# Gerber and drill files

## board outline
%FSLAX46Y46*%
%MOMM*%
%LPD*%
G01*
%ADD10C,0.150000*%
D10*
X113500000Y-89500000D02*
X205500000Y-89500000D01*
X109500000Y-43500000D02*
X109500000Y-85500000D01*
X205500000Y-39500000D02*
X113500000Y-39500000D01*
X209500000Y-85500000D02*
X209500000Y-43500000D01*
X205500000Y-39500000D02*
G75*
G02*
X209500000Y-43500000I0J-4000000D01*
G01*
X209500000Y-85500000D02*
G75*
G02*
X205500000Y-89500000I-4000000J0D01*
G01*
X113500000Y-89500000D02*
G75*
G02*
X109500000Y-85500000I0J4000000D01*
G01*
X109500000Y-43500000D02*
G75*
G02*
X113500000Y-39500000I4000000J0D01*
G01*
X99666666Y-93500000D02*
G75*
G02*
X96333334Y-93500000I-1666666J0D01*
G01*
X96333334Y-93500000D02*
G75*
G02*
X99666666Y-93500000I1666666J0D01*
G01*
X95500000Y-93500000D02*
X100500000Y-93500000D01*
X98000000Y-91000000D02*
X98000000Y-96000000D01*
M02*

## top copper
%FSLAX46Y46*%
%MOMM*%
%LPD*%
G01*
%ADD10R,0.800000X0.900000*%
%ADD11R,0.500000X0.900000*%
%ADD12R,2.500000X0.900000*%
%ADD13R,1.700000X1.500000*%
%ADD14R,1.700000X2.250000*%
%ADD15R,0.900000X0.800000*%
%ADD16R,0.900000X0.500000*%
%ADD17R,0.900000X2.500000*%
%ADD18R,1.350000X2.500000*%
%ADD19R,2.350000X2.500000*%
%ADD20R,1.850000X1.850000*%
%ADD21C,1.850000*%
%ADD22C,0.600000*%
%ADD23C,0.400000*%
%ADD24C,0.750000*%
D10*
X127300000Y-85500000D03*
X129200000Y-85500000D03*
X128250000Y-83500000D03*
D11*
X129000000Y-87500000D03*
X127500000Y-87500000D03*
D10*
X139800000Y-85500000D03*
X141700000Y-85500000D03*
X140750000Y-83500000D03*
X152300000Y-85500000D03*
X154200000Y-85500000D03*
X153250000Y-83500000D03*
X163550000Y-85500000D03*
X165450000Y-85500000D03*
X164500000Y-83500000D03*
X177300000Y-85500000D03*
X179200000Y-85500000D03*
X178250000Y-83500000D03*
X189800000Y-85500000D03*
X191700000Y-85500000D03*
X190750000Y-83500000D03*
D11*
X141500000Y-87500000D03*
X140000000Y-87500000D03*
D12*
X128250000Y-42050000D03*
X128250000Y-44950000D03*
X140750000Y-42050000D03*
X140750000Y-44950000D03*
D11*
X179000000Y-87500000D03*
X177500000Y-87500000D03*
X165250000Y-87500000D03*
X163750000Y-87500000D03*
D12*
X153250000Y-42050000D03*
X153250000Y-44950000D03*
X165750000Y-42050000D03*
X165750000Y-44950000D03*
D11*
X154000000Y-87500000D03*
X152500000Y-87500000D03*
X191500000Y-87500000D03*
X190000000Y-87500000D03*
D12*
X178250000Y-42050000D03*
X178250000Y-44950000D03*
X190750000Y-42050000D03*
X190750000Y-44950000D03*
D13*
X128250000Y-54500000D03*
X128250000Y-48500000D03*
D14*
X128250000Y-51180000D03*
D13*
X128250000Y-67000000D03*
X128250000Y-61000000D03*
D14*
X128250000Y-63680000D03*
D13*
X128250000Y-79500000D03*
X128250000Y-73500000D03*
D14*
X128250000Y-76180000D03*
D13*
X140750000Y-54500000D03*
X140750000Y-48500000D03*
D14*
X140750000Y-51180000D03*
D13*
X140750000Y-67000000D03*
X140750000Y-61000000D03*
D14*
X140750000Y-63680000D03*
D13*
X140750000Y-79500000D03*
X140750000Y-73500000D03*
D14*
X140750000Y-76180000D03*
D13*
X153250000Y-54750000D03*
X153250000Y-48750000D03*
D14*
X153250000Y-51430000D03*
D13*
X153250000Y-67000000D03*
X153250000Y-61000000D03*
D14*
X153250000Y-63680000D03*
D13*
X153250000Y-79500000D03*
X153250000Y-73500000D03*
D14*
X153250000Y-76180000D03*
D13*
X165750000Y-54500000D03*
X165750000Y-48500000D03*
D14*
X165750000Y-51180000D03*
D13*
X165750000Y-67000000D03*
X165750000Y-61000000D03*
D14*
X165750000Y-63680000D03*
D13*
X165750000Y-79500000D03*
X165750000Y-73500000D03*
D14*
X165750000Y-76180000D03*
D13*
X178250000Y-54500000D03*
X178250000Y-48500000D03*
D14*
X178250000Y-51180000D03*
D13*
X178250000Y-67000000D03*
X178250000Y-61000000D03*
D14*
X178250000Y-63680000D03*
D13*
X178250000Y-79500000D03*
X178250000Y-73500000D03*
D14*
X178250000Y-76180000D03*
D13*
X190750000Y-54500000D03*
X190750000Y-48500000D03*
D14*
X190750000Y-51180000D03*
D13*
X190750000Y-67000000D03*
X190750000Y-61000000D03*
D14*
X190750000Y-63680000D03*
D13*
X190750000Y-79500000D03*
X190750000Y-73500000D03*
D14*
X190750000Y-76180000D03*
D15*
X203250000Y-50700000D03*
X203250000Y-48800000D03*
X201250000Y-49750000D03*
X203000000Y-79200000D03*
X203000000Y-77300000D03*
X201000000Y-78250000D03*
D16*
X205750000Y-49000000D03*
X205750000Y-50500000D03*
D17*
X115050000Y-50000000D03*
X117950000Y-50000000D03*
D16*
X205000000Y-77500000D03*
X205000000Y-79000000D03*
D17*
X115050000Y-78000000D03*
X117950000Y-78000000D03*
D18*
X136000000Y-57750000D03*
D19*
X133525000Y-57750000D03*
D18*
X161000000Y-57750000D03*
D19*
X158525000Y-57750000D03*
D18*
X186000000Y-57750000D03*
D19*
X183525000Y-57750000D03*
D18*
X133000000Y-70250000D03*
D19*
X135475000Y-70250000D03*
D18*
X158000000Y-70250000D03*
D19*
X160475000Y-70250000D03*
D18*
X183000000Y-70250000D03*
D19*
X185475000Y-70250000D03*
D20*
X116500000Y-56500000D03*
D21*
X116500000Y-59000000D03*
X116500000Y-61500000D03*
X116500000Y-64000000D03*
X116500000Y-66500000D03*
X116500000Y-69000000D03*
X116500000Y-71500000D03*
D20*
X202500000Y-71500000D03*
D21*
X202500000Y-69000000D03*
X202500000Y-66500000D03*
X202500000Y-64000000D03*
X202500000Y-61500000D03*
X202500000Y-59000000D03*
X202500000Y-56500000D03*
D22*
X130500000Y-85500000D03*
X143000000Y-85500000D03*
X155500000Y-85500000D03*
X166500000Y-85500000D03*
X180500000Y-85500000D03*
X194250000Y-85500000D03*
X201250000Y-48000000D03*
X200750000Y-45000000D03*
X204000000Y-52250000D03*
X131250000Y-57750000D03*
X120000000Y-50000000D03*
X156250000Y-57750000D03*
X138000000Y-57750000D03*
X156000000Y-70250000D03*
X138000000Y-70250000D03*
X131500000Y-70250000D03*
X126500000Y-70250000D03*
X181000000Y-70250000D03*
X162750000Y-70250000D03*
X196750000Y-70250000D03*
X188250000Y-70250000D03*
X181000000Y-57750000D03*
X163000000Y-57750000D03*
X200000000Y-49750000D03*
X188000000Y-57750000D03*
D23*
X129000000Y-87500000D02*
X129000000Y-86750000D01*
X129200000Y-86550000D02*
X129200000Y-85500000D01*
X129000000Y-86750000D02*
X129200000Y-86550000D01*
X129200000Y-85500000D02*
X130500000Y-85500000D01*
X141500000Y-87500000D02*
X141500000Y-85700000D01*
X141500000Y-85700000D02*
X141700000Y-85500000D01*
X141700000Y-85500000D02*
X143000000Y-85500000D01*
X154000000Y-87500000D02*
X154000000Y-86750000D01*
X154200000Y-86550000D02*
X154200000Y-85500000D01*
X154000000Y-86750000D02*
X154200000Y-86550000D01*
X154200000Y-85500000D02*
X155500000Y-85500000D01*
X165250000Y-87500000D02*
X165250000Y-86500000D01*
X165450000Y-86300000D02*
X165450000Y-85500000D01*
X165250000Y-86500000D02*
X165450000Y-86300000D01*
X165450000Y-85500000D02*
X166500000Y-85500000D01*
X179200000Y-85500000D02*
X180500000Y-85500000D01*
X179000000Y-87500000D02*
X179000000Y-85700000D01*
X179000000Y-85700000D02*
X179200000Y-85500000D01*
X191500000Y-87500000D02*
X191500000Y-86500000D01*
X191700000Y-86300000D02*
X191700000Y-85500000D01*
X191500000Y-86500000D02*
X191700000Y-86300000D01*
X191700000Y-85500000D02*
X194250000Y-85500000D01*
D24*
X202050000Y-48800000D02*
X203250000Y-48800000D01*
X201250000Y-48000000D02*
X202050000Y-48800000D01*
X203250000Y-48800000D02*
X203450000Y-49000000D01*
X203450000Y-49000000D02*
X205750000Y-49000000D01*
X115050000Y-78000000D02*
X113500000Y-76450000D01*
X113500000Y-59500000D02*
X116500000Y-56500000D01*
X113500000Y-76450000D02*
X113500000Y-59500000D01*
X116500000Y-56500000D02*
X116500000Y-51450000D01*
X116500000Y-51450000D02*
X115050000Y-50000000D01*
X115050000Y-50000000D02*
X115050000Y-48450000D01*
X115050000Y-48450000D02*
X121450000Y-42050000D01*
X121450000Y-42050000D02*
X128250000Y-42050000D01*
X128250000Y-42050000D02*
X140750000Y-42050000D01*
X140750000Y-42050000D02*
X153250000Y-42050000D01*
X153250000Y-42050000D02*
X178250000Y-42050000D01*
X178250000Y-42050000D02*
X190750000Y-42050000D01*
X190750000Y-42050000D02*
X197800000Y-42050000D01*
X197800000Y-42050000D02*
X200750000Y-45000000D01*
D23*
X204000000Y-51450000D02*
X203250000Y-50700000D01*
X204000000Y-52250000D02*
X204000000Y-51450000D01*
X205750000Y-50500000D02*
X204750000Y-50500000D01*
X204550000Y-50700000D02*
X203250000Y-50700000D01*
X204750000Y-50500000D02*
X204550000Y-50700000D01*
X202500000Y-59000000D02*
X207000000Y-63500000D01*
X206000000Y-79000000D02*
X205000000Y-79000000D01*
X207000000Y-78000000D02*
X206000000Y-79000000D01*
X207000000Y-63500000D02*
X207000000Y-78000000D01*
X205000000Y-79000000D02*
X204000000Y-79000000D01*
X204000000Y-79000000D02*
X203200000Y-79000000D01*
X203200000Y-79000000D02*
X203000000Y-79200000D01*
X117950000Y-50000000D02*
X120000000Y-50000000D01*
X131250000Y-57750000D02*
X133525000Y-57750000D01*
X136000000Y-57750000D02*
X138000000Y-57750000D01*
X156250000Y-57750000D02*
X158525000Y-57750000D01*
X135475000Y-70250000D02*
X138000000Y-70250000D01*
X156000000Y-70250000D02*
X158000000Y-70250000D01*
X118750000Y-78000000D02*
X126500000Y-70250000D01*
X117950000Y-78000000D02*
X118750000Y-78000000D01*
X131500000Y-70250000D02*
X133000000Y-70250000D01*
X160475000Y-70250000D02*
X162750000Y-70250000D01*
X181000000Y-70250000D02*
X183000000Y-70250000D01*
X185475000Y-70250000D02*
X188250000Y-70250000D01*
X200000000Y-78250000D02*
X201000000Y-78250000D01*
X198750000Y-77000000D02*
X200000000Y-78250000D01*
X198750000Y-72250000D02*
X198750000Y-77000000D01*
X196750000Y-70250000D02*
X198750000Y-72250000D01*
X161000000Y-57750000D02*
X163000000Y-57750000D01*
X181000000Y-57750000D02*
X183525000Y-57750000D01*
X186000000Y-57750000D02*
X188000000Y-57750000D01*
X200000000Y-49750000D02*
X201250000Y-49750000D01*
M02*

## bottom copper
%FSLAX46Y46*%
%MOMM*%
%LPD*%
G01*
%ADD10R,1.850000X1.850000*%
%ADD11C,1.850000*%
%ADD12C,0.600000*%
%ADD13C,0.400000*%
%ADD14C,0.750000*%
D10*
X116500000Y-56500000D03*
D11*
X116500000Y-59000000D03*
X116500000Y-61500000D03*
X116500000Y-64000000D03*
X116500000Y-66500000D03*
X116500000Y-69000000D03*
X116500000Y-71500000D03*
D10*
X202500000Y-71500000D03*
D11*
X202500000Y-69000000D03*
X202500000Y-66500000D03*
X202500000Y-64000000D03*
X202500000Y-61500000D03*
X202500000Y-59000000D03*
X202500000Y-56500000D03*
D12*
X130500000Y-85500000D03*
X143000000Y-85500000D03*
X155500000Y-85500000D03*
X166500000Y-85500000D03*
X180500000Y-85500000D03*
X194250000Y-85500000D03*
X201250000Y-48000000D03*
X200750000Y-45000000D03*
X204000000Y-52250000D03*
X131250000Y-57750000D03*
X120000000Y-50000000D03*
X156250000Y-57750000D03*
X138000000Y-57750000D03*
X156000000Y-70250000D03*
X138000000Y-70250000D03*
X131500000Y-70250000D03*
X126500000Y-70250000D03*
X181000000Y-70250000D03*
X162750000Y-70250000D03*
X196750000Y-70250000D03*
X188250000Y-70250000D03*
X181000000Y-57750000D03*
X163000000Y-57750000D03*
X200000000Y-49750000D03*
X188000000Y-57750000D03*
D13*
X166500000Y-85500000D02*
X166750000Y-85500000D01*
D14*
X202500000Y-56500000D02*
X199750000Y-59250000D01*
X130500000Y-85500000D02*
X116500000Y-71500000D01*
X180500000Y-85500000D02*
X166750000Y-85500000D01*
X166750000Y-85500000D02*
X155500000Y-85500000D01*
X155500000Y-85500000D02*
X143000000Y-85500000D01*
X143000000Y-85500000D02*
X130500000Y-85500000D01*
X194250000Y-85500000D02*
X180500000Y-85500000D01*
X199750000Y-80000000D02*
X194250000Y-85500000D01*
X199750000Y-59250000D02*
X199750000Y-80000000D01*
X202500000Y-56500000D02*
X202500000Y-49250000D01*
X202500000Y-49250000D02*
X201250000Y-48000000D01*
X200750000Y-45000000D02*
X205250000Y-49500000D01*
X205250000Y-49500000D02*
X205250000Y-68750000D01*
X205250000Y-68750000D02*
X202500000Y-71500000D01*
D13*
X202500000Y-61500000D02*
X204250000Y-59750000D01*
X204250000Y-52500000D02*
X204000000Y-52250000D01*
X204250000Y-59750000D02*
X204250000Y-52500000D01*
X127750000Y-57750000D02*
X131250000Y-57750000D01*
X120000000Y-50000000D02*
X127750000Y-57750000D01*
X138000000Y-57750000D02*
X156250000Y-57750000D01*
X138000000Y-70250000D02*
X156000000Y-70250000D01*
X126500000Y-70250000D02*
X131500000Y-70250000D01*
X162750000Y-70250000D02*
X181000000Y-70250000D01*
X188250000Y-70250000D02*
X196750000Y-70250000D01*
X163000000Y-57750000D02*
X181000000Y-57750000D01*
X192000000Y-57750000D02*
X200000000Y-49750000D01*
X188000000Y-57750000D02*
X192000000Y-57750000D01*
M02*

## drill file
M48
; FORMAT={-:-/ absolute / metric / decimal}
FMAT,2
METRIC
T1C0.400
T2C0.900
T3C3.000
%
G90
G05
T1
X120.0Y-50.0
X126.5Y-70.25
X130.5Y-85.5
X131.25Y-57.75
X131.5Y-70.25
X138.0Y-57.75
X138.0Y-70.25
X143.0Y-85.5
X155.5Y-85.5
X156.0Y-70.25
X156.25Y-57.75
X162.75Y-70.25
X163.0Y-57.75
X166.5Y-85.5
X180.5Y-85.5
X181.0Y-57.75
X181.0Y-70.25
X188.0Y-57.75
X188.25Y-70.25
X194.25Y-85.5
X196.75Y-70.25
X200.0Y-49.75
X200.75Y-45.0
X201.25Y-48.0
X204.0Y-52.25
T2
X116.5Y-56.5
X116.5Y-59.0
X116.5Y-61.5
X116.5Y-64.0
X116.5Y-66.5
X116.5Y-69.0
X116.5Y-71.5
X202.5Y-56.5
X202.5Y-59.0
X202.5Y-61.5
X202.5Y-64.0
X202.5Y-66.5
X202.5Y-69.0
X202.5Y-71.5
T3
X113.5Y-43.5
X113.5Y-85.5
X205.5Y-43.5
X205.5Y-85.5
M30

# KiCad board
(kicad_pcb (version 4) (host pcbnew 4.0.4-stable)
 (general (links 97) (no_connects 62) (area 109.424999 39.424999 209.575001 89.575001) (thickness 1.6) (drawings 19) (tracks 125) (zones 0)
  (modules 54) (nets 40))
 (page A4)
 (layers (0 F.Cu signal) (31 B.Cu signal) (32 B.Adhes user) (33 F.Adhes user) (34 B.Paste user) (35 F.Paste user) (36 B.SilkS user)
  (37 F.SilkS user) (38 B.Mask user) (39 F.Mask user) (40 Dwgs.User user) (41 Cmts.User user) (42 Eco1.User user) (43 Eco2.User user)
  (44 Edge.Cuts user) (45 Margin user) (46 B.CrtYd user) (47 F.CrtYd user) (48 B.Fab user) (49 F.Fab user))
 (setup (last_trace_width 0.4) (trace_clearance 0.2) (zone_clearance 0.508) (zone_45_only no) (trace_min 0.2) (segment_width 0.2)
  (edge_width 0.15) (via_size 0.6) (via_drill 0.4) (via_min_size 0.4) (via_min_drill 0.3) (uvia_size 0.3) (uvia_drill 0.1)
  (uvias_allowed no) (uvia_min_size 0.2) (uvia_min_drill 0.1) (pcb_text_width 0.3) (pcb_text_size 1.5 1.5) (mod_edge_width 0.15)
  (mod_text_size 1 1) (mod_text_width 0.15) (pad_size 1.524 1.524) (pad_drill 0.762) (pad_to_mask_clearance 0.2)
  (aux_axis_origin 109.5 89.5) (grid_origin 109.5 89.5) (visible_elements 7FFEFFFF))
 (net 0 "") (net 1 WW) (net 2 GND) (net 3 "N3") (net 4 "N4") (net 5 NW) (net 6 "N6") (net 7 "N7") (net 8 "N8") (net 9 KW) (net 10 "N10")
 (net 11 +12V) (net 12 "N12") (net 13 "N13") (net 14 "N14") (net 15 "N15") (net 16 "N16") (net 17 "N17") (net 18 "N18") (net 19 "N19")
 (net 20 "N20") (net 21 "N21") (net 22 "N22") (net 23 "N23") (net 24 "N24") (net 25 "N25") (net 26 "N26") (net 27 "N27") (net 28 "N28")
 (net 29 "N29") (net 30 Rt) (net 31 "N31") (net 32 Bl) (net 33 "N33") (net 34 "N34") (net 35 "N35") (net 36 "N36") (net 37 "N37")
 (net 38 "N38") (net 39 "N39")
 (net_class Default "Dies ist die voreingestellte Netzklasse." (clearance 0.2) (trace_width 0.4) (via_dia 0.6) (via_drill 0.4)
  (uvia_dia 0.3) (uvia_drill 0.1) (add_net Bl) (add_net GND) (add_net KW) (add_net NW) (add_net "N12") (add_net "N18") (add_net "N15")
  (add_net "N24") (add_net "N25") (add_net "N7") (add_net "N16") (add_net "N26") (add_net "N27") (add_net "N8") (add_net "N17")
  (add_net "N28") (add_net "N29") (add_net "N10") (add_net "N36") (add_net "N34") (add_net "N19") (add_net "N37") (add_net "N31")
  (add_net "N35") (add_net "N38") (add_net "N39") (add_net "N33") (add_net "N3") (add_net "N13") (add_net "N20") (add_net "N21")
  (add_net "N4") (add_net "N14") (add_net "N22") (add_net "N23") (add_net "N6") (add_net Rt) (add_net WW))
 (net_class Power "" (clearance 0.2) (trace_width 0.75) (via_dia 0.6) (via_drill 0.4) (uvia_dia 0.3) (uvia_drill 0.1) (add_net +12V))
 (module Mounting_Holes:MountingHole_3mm (layer F.Cu) (at 205.5 85.5)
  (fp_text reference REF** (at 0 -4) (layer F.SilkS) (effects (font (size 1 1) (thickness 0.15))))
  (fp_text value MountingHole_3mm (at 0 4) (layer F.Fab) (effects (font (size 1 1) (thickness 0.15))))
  (pad 1 np_thru_hole circle (at 0 0) (size 3 3) (drill 3) (layers *.Cu *.Mask)))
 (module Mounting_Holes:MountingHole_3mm (layer F.Cu) (at 205.5 43.5)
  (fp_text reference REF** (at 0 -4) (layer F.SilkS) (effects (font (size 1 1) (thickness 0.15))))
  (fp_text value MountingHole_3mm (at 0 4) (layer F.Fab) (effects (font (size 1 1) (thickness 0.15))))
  (pad 1 np_thru_hole circle (at 0 0) (size 3 3) (drill 3) (layers *.Cu *.Mask)))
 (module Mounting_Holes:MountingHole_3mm (layer F.Cu) (at 113.5 85.5)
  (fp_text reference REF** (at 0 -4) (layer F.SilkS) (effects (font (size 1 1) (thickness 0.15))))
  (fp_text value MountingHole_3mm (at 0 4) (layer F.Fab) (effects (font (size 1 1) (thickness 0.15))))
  (pad 1 np_thru_hole circle (at 0 0) (size 3 3) (drill 3) (layers *.Cu *.Mask)))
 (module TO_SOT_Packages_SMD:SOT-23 (layer F.Cu) (at 128.25 84.5 90)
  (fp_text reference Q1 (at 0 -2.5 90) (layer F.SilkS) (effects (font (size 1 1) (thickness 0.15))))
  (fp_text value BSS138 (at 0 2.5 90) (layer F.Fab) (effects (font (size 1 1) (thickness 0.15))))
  (pad 1 smd rect (at -1 -0.95 90) (size 0.9 0.8) (layers F.Cu F.Paste F.Mask) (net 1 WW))
  (pad 2 smd rect (at -1 0.95 90) (size 0.9 0.8) (layers F.Cu F.Paste F.Mask) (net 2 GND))
  (pad 3 smd rect (at 1 0 90) (size 0.9 0.8) (layers F.Cu F.Paste F.Mask) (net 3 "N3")))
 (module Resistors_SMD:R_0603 (layer F.Cu) (at 128.25 87.5 180)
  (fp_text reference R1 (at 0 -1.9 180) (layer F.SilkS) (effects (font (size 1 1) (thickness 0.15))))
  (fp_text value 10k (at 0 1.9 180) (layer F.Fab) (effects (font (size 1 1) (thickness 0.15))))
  (pad 1 smd rect (at -0.75 0 180) (size 0.5 0.9) (layers F.Cu F.Paste F.Mask) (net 2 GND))
  (pad 2 smd rect (at 0.75 0 180) (size 0.5 0.9) (layers F.Cu F.Paste F.Mask) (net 1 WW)))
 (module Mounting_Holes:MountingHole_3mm (layer F.Cu) (at 113.5 43.5)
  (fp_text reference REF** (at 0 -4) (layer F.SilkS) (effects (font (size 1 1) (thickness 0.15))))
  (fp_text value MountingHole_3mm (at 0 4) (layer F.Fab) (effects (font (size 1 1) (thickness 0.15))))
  (pad 1 np_thru_hole circle (at 0 0) (size 3 3) (drill 3) (layers *.Cu *.Mask)))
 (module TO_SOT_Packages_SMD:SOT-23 (layer F.Cu) (at 140.75 84.5 90)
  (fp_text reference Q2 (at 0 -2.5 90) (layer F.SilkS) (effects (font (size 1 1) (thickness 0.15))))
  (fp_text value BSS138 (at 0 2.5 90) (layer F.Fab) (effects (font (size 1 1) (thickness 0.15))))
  (pad 1 smd rect (at -1 -0.95 90) (size 0.9 0.8) (layers F.Cu F.Paste F.Mask) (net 1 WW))
  (pad 2 smd rect (at -1 0.95 90) (size 0.9 0.8) (layers F.Cu F.Paste F.Mask) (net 2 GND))
  (pad 3 smd rect (at 1 0 90) (size 0.9 0.8) (layers F.Cu F.Paste F.Mask) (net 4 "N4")))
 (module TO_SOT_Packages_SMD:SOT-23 (layer F.Cu) (at 153.25 84.5 90)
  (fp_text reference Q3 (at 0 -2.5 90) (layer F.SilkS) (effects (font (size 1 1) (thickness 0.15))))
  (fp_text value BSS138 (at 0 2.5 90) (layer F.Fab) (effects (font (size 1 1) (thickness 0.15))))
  (pad 1 smd rect (at -1 -0.95 90) (size 0.9 0.8) (layers F.Cu F.Paste F.Mask) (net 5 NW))
  (pad 2 smd rect (at -1 0.95 90) (size 0.9 0.8) (layers F.Cu F.Paste F.Mask) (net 2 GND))
  (pad 3 smd rect (at 1 0 90) (size 0.9 0.8) (layers F.Cu F.Paste F.Mask) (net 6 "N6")))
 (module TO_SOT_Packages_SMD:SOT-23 (layer F.Cu) (at 164.5 84.5 90)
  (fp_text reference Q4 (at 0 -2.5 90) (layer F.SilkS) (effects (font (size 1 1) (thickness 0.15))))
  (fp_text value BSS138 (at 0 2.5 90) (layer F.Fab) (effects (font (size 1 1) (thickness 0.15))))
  (pad 1 smd rect (at -1 -0.95 90) (size 0.9 0.8) (layers F.Cu F.Paste F.Mask) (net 5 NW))
  (pad 2 smd rect (at -1 0.95 90) (size 0.9 0.8) (layers F.Cu F.Paste F.Mask) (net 2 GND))
  (pad 3 smd rect (at 1 0 90) (size 0.9 0.8) (layers F.Cu F.Paste F.Mask) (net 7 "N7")))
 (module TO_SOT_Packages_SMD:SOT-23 (layer F.Cu) (at 178.25 84.5 90)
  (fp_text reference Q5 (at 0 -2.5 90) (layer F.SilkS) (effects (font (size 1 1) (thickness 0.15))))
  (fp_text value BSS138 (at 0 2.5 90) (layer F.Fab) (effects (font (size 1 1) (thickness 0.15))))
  (pad 1 smd rect (at -1 -0.95 90) (size 0.9 0.8) (layers F.Cu F.Paste F.Mask) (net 5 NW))
  (pad 2 smd rect (at -1 0.95 90) (size 0.9 0.8) (layers F.Cu F.Paste F.Mask) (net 2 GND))
  (pad 3 smd rect (at 1 0 90) (size 0.9 0.8) (layers F.Cu F.Paste F.Mask) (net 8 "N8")))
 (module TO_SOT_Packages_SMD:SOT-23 (layer F.Cu) (at 190.75 84.5 90)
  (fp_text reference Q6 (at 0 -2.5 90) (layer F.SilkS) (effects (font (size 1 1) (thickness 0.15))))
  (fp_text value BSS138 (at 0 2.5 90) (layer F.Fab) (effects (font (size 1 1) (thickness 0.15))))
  (pad 1 smd rect (at -1 -0.95 90) (size 0.9 0.8) (layers F.Cu F.Paste F.Mask) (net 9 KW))
  (pad 2 smd rect (at -1 0.95 90) (size 0.9 0.8) (layers F.Cu F.Paste F.Mask) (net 2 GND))
  (pad 3 smd rect (at 1 0 90) (size 0.9 0.8) (layers F.Cu F.Paste F.Mask) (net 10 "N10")))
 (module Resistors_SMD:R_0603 (layer F.Cu) (at 140.75 87.5 180)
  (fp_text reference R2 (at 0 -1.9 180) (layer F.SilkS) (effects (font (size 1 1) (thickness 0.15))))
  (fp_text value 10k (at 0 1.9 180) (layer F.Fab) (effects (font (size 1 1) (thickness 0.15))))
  (pad 1 smd rect (at -0.75 0 180) (size 0.5 0.9) (layers F.Cu F.Paste F.Mask) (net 2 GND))
  (pad 2 smd rect (at 0.75 0 180) (size 0.5 0.9) (layers F.Cu F.Paste F.Mask) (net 1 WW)))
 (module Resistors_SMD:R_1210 (layer F.Cu) (at 128.25 43.5 270)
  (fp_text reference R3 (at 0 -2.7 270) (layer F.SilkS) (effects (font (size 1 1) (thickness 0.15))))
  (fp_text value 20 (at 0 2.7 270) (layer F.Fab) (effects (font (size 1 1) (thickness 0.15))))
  (pad 1 smd rect (at -1.45 0 270) (size 0.9 2.5) (layers F.Cu F.Paste F.Mask) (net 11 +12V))
  (pad 2 smd rect (at 1.45 0 270) (size 0.9 2.5) (layers F.Cu F.Paste F.Mask) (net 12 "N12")))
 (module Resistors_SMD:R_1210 (layer F.Cu) (at 140.75 43.5 270)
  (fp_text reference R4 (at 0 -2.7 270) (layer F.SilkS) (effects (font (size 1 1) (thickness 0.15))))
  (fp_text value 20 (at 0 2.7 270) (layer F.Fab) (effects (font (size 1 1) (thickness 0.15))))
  (pad 1 smd rect (at -1.45 0 270) (size 0.9 2.5) (layers F.Cu F.Paste F.Mask) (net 11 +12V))
  (pad 2 smd rect (at 1.45 0 270) (size 0.9 2.5) (layers F.Cu F.Paste F.Mask) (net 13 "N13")))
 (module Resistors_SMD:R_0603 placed (layer F.Cu) (at 178.25 87.5 180)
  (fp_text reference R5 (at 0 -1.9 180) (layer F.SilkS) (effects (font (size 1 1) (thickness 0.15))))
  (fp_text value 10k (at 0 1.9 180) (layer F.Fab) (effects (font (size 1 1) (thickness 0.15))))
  (pad 1 smd rect (at -0.75 0 180) (size 0.5 0.9) (layers F.Cu F.Paste F.Mask) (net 2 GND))
  (pad 2 smd rect (at 0.75 0 180) (size 0.5 0.9) (layers F.Cu F.Paste F.Mask) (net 5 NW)))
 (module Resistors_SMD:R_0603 (layer F.Cu) (at 164.5 87.5 180)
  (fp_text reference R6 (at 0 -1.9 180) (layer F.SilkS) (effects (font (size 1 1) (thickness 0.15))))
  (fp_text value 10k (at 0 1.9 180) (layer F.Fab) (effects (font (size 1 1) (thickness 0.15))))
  (pad 1 smd rect (at -0.75 0 180) (size 0.5 0.9) (layers F.Cu F.Paste F.Mask) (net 2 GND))
  (pad 2 smd rect (at 0.75 0 180) (size 0.5 0.9) (layers F.Cu F.Paste F.Mask) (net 5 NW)))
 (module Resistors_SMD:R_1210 (layer F.Cu) (at 153.25 43.5 270)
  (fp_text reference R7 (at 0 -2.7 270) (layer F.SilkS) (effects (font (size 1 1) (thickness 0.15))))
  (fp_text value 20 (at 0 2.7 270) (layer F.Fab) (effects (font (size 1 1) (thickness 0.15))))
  (pad 1 smd rect (at -1.45 0 270) (size 0.9 2.5) (layers F.Cu F.Paste F.Mask) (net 11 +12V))
  (pad 2 smd rect (at 1.45 0 270) (size 0.9 2.5) (layers F.Cu F.Paste F.Mask) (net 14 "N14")))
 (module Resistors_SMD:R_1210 (layer F.Cu) (at 165.75 43.5 270)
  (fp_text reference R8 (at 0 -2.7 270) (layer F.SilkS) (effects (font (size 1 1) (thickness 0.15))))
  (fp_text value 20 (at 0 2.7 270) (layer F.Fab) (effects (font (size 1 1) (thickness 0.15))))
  (pad 1 smd rect (at -1.45 0 270) (size 0.9 2.5) (layers F.Cu F.Paste F.Mask) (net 11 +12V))
  (pad 2 smd rect (at 1.45 0 270) (size 0.9 2.5) (layers F.Cu F.Paste F.Mask) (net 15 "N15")))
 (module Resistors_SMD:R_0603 (layer F.Cu) (at 153.25 87.5 180)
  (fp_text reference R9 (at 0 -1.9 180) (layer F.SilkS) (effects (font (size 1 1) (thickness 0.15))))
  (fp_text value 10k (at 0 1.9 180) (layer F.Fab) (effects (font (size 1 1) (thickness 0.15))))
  (pad 1 smd rect (at -0.75 0 180) (size 0.5 0.9) (layers F.Cu F.Paste F.Mask) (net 2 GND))
  (pad 2 smd rect (at 0.75 0 180) (size 0.5 0.9) (layers F.Cu F.Paste F.Mask) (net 5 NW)))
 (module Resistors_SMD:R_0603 (layer F.Cu) (at 190.75 87.5 180)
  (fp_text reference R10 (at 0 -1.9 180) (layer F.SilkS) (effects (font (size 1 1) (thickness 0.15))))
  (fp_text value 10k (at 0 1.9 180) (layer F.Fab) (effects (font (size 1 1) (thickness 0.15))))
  (pad 1 smd rect (at -0.75 0 180) (size 0.5 0.9) (layers F.Cu F.Paste F.Mask) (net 2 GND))
  (pad 2 smd rect (at 0.75 0 180) (size 0.5 0.9) (layers F.Cu F.Paste F.Mask) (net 9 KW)))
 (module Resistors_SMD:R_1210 (layer F.Cu) (at 178.25 43.5 270)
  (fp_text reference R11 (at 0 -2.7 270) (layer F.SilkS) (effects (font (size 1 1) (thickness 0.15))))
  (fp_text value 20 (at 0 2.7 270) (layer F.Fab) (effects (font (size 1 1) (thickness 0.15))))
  (pad 1 smd rect (at -1.45 0 270) (size 0.9 2.5) (layers F.Cu F.Paste F.Mask) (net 11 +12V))
  (pad 2 smd rect (at 1.45 0 270) (size 0.9 2.5) (layers F.Cu F.Paste F.Mask) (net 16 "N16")))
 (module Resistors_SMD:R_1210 (layer F.Cu) (at 190.75 43.5 270)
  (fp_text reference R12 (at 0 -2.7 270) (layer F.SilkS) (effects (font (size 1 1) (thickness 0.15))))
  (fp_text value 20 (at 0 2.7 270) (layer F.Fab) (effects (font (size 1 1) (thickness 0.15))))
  (pad 1 smd rect (at -1.45 0 270) (size 0.9 2.5) (layers F.Cu F.Paste F.Mask) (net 11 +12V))
  (pad 2 smd rect (at 1.45 0 270) (size 0.9 2.5) (layers F.Cu F.Paste F.Mask) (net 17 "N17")))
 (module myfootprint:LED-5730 (layer F.Cu) (at 128.25 51.5 90)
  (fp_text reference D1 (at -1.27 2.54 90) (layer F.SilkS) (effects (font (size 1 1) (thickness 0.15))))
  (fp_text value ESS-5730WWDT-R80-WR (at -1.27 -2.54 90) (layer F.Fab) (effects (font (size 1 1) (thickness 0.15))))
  (pad 2 smd rect (at -3 0 90) (size 1.5 1.7) (layers F.Cu F.Paste F.Mask) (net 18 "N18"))
  (pad 1 smd rect (at 3 0 90) (size 1.5 1.7) (layers F.Cu F.Paste F.Mask) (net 12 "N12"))
  (pad 1 smd rect (at 0.32 0 90) (size 2.25 1.7) (layers F.Cu F.Paste F.Mask) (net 12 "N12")))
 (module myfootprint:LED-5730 (layer F.Cu) (at 128.25 64 90)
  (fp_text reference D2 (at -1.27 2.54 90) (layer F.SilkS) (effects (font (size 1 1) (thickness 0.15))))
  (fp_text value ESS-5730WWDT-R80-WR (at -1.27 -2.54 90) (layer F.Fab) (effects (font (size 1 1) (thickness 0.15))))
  (pad 2 smd rect (at -3 0 90) (size 1.5 1.7) (layers F.Cu F.Paste F.Mask) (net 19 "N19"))
  (pad 1 smd rect (at 3 0 90) (size 1.5 1.7) (layers F.Cu F.Paste F.Mask) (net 18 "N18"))
  (pad 1 smd rect (at 0.32 0 90) (size 2.25 1.7) (layers F.Cu F.Paste F.Mask) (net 18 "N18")))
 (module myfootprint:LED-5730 (layer F.Cu) (at 128.25 76.5 90)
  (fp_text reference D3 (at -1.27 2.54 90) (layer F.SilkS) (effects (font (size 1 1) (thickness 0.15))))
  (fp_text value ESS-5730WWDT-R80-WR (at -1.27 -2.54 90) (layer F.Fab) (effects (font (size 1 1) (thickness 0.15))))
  (pad 2 smd rect (at -3 0 90) (size 1.5 1.7) (layers F.Cu F.Paste F.Mask) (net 3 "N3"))
  (pad 1 smd rect (at 3 0 90) (size 1.5 1.7) (layers F.Cu F.Paste F.Mask) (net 19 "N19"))
  (pad 1 smd rect (at 0.32 0 90) (size 2.25 1.7) (layers F.Cu F.Paste F.Mask) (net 19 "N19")))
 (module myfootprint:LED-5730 (layer F.Cu) (at 140.75 51.5 90)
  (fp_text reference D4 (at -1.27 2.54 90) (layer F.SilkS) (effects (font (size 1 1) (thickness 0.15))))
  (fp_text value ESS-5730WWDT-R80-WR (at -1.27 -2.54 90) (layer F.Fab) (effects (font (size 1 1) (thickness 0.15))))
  (pad 2 smd rect (at -3 0 90) (size 1.5 1.7) (layers F.Cu F.Paste F.Mask) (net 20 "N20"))
  (pad 1 smd rect (at 3 0 90) (size 1.5 1.7) (layers F.Cu F.Paste F.Mask) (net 13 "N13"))
  (pad 1 smd rect (at 0.32 0 90) (size 2.25 1.7) (layers F.Cu F.Paste F.Mask) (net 13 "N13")))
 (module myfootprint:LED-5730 (layer F.Cu) (at 140.75 64 90)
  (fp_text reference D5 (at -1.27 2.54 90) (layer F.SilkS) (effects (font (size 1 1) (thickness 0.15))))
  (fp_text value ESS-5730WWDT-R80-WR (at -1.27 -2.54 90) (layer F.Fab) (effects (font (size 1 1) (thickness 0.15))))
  (pad 2 smd rect (at -3 0 90) (size 1.5 1.7) (layers F.Cu F.Paste F.Mask) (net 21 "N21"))
  (pad 1 smd rect (at 3 0 90) (size 1.5 1.7) (layers F.Cu F.Paste F.Mask) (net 20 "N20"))
  (pad 1 smd rect (at 0.32 0 90) (size 2.25 1.7) (layers F.Cu F.Paste F.Mask) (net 20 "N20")))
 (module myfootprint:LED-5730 (layer F.Cu) (at 140.75 76.5 90)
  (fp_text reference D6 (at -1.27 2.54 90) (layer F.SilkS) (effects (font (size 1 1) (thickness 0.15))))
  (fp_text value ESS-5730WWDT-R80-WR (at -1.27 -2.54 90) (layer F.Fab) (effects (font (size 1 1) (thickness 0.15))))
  (pad 2 smd rect (at -3 0 90) (size 1.5 1.7) (layers F.Cu F.Paste F.Mask) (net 4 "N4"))
  (pad 1 smd rect (at 3 0 90) (size 1.5 1.7) (layers F.Cu F.Paste F.Mask) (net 21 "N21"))
  (pad 1 smd rect (at 0.32 0 90) (size 2.25 1.7) (layers F.Cu F.Paste F.Mask) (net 21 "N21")))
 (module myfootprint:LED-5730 (layer F.Cu) (at 153.25 51.75 90)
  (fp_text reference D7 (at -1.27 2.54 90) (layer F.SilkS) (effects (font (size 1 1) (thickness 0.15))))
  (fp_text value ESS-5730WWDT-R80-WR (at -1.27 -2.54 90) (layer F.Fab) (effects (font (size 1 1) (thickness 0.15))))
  (pad 2 smd rect (at -3 0 90) (size 1.5 1.7) (layers F.Cu F.Paste F.Mask) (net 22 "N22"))
  (pad 1 smd rect (at 3 0 90) (size 1.5 1.7) (layers F.Cu F.Paste F.Mask) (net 14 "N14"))
  (pad 1 smd rect (at 0.32 0 90) (size 2.25 1.7) (layers F.Cu F.Paste F.Mask) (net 14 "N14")))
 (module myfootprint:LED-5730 (layer F.Cu) (at 153.25 64 90)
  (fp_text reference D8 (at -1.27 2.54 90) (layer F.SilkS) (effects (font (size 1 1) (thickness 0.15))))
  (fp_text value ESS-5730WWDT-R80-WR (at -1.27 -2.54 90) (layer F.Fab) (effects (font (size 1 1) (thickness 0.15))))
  (pad 2 smd rect (at -3 0 90) (size 1.5 1.7) (layers F.Cu F.Paste F.Mask) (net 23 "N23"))
  (pad 1 smd rect (at 3 0 90) (size 1.5 1.7) (layers F.Cu F.Paste F.Mask) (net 22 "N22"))
  (pad 1 smd rect (at 0.32 0 90) (size 2.25 1.7) (layers F.Cu F.Paste F.Mask) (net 22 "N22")))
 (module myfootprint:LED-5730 (layer F.Cu) (at 153.25 76.5 90)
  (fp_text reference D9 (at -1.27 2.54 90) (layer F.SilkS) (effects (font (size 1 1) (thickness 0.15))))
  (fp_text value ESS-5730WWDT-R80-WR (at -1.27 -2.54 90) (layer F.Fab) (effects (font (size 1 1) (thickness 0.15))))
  (pad 2 smd rect (at -3 0 90) (size 1.5 1.7) (layers F.Cu F.Paste F.Mask) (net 6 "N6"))
  (pad 1 smd rect (at 3 0 90) (size 1.5 1.7) (layers F.Cu F.Paste F.Mask) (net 23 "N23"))
  (pad 1 smd rect (at 0.32 0 90) (size 2.25 1.7) (layers F.Cu F.Paste F.Mask) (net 23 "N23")))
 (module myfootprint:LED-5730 (layer F.Cu) (at 165.75 51.5 90)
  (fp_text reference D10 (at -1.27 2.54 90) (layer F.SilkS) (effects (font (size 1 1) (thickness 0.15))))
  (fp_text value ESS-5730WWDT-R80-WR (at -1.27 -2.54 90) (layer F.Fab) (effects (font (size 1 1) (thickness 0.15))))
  (pad 2 smd rect (at -3 0 90) (size 1.5 1.7) (layers F.Cu F.Paste F.Mask) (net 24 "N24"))
  (pad 1 smd rect (at 3 0 90) (size 1.5 1.7) (layers F.Cu F.Paste F.Mask) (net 15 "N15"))
  (pad 1 smd rect (at 0.32 0 90) (size 2.25 1.7) (layers F.Cu F.Paste F.Mask) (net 15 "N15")))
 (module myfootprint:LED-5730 (layer F.Cu) (at 165.75 64 90)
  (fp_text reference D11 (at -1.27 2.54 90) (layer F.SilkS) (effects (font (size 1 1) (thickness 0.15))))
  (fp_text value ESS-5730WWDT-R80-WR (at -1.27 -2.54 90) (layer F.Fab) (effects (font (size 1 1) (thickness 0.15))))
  (pad 2 smd rect (at -3 0 90) (size 1.5 1.7) (layers F.Cu F.Paste F.Mask) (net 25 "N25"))
  (pad 1 smd rect (at 3 0 90) (size 1.5 1.7) (layers F.Cu F.Paste F.Mask) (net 24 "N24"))
  (pad 1 smd rect (at 0.32 0 90) (size 2.25 1.7) (layers F.Cu F.Paste F.Mask) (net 24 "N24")))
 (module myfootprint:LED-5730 (layer F.Cu) (at 165.75 76.5 90)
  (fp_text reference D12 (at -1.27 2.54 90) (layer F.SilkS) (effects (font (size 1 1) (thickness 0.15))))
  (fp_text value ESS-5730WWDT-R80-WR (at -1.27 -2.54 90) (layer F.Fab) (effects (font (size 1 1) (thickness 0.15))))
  (pad 2 smd rect (at -3 0 90) (size 1.5 1.7) (layers F.Cu F.Paste F.Mask) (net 7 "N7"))
  (pad 1 smd rect (at 3 0 90) (size 1.5 1.7) (layers F.Cu F.Paste F.Mask) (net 25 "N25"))
  (pad 1 smd rect (at 0.32 0 90) (size 2.25 1.7) (layers F.Cu F.Paste F.Mask) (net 25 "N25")))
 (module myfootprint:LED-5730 (layer F.Cu) (at 178.25 51.5 90)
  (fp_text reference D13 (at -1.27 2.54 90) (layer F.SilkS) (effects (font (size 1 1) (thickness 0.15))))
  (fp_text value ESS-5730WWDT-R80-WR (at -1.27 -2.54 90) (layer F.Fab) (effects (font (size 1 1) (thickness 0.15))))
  (pad 2 smd rect (at -3 0 90) (size 1.5 1.7) (layers F.Cu F.Paste F.Mask) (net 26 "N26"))
  (pad 1 smd rect (at 3 0 90) (size 1.5 1.7) (layers F.Cu F.Paste F.Mask) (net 16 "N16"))
  (pad 1 smd rect (at 0.32 0 90) (size 2.25 1.7) (layers F.Cu F.Paste F.Mask) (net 16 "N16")))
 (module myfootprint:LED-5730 (layer F.Cu) (at 178.25 64 90)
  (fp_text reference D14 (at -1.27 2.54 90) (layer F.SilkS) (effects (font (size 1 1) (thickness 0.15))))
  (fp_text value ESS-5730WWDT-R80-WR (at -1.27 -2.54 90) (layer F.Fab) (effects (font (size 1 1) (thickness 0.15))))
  (pad 2 smd rect (at -3 0 90) (size 1.5 1.7) (layers F.Cu F.Paste F.Mask) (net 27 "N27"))
  (pad 1 smd rect (at 3 0 90) (size 1.5 1.7) (layers F.Cu F.Paste F.Mask) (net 26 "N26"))
  (pad 1 smd rect (at 0.32 0 90) (size 2.25 1.7) (layers F.Cu F.Paste F.Mask) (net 26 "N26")))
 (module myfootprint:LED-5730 (layer F.Cu) (at 178.25 76.5 90)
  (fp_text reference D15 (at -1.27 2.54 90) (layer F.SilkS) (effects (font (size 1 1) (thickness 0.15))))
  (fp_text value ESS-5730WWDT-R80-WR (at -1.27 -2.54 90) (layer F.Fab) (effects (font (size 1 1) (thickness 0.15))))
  (pad 2 smd rect (at -3 0 90) (size 1.5 1.7) (layers F.Cu F.Paste F.Mask) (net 8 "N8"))
  (pad 1 smd rect (at 3 0 90) (size 1.5 1.7) (layers F.Cu F.Paste F.Mask) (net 27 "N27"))
  (pad 1 smd rect (at 0.32 0 90) (size 2.25 1.7) (layers F.Cu F.Paste F.Mask) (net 27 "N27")))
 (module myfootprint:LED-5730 (layer F.Cu) (at 190.75 51.5 90)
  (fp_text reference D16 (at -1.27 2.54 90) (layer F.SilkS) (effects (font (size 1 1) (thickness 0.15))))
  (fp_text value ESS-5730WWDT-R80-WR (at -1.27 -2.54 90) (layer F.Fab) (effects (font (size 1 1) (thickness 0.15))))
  (pad 2 smd rect (at -3 0 90) (size 1.5 1.7) (layers F.Cu F.Paste F.Mask) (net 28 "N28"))
  (pad 1 smd rect (at 3 0 90) (size 1.5 1.7) (layers F.Cu F.Paste F.Mask) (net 17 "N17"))
  (pad 1 smd rect (at 0.32 0 90) (size 2.25 1.7) (layers F.Cu F.Paste F.Mask) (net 17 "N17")))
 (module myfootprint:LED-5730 (layer F.Cu) (at 190.75 64 90)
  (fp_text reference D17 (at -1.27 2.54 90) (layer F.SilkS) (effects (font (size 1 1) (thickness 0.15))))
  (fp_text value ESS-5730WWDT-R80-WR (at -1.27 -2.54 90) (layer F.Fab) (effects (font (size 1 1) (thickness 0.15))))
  (pad 2 smd rect (at -3 0 90) (size 1.5 1.7) (layers F.Cu F.Paste F.Mask) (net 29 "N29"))
  (pad 1 smd rect (at 3 0 90) (size 1.5 1.7) (layers F.Cu F.Paste F.Mask) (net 28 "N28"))
  (pad 1 smd rect (at 0.32 0 90) (size 2.25 1.7) (layers F.Cu F.Paste F.Mask) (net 28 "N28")))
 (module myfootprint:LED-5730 (layer F.Cu) (at 190.75 76.5 90)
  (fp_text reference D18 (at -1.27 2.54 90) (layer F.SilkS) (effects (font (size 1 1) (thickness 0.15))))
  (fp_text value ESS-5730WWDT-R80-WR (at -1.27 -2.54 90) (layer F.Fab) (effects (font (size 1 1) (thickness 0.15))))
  (pad 2 smd rect (at -3 0 90) (size 1.5 1.7) (layers F.Cu F.Paste F.Mask) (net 10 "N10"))
  (pad 1 smd rect (at 3 0 90) (size 1.5 1.7) (layers F.Cu F.Paste F.Mask) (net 29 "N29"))
  (pad 1 smd rect (at 0.32 0 90) (size 2.25 1.7) (layers F.Cu F.Paste F.Mask) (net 29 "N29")))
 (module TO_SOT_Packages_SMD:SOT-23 (layer F.Cu) (at 202.25 49.75 180)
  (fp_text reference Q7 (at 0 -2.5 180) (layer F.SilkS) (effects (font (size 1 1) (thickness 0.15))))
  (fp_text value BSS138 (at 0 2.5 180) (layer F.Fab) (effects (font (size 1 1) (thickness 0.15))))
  (pad 1 smd rect (at -1 -0.95 180) (size 0.9 0.8) (layers F.Cu F.Paste F.Mask) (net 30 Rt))
  (pad 2 smd rect (at -1 0.95 180) (size 0.9 0.8) (layers F.Cu F.Paste F.Mask) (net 2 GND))
  (pad 3 smd rect (at 1 0 180) (size 0.9 0.8) (layers F.Cu F.Paste F.Mask) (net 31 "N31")))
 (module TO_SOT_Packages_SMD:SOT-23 (layer F.Cu) (at 202 78.25 180)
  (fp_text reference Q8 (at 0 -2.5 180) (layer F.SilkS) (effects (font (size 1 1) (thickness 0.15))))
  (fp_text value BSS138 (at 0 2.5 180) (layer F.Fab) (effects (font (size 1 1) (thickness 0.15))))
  (pad 1 smd rect (at -1 -0.95 180) (size 0.9 0.8) (layers F.Cu F.Paste F.Mask) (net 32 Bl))
  (pad 2 smd rect (at -1 0.95 180) (size 0.9 0.8) (layers F.Cu F.Paste F.Mask) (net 2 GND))
  (pad 3 smd rect (at 1 0 180) (size 0.9 0.8) (layers F.Cu F.Paste F.Mask) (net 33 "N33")))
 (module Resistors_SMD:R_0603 (layer F.Cu) (at 205.75 49.75 270)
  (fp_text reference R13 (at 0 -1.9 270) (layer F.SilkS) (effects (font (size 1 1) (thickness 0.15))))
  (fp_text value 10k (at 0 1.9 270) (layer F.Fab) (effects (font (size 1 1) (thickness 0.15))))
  (pad 1 smd rect (at -0.75 0 270) (size 0.5 0.9) (layers F.Cu F.Paste F.Mask) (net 2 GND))
  (pad 2 smd rect (at 0.75 0 270) (size 0.5 0.9) (layers F.Cu F.Paste F.Mask) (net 30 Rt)))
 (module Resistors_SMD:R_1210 (layer F.Cu) (at 116.5 50)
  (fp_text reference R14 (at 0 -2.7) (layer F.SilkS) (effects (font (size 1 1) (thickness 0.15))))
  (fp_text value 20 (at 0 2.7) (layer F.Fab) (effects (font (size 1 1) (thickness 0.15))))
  (pad 1 smd rect (at -1.45 0) (size 0.9 2.5) (layers F.Cu F.Paste F.Mask) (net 11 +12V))
  (pad 2 smd rect (at 1.45 0) (size 0.9 2.5) (layers F.Cu F.Paste F.Mask) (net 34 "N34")))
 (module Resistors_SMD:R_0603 (layer F.Cu) (at 205 78.25 270)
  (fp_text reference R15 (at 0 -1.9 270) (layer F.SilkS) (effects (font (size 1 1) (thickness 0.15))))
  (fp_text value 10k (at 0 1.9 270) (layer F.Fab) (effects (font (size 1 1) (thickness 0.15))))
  (pad 1 smd rect (at -0.75 0 270) (size 0.5 0.9) (layers F.Cu F.Paste F.Mask) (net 2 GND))
  (pad 2 smd rect (at 0.75 0 270) (size 0.5 0.9) (layers F.Cu F.Paste F.Mask) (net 32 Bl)))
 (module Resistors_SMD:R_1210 (layer F.Cu) (at 116.5 78)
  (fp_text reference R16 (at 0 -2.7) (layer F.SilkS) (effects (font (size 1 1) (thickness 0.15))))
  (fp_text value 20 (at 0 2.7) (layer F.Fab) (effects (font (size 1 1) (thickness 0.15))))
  (pad 1 smd rect (at -1.45 0) (size 0.9 2.5) (layers F.Cu F.Paste F.Mask) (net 11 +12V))
  (pad 2 smd rect (at 1.45 0) (size 0.9 2.5) (layers F.Cu F.Paste F.Mask) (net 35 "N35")))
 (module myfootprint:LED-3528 (layer F.Cu) (at 134.5 57.75 180)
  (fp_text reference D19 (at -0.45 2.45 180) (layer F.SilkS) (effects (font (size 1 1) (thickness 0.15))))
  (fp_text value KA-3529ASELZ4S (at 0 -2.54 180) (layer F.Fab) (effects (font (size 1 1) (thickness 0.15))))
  (pad 1 smd rect (at -1.5 0 180) (size 1.35 2.5) (layers F.Cu F.Paste F.Mask) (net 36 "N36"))
  (pad 2 smd rect (at 0.975 0 180) (size 2.35 2.5) (layers F.Cu F.Paste F.Mask) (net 34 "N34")))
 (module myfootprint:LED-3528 (layer F.Cu) (at 159.5 57.75 180)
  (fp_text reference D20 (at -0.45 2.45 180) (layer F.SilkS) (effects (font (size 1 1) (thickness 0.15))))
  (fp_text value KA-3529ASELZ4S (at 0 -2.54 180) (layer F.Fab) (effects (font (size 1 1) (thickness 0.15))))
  (pad 1 smd rect (at -1.5 0 180) (size 1.35 2.5) (layers F.Cu F.Paste F.Mask) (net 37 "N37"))
  (pad 2 smd rect (at 0.975 0 180) (size 2.35 2.5) (layers F.Cu F.Paste F.Mask) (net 36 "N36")))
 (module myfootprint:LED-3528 (layer F.Cu) (at 184.5 57.75 180)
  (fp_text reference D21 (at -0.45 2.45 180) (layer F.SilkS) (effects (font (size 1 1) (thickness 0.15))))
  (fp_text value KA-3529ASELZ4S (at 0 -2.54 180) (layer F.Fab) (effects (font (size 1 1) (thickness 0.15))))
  (pad 1 smd rect (at -1.5 0 180) (size 1.35 2.5) (layers F.Cu F.Paste F.Mask) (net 31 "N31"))
  (pad 2 smd rect (at 0.975 0 180) (size 2.35 2.5) (layers F.Cu F.Paste F.Mask) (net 37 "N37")))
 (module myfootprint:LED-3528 (layer F.Cu) (at 134.5 70.25)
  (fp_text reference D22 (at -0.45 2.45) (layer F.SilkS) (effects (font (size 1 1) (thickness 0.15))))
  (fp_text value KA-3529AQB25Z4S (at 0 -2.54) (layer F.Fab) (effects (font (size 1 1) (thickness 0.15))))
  (pad 1 smd rect (at -1.5 0) (size 1.35 2.5) (layers F.Cu F.Paste F.Mask) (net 35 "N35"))
  (pad 2 smd rect (at 0.975 0) (size 2.35 2.5) (layers F.Cu F.Paste F.Mask) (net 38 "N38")))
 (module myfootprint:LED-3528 (layer F.Cu) (at 159.5 70.25)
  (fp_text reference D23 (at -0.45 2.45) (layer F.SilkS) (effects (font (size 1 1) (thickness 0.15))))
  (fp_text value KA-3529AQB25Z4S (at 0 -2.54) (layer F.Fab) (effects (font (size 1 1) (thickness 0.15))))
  (pad 1 smd rect (at -1.5 0) (size 1.35 2.5) (layers F.Cu F.Paste F.Mask) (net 38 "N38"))
  (pad 2 smd rect (at 0.975 0) (size 2.35 2.5) (layers F.Cu F.Paste F.Mask) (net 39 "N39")))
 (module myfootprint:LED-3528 (layer F.Cu) (at 184.5 70.25)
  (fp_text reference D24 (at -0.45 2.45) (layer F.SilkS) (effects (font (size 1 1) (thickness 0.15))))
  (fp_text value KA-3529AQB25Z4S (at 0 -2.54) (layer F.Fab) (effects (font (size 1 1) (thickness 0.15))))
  (pad 1 smd rect (at -1.5 0) (size 1.35 2.5) (layers F.Cu F.Paste F.Mask) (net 39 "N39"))
  (pad 2 smd rect (at 0.975 0) (size 2.35 2.5) (layers F.Cu F.Paste F.Mask) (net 33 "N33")))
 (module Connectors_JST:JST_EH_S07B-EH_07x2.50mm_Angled (layer B.Cu) (at 116.5 56.5 270)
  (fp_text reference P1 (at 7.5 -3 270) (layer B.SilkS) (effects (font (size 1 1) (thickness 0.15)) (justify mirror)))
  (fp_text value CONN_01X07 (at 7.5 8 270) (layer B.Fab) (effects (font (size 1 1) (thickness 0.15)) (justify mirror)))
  (pad 1 thru_hole rect (at 0 0 270) (size 1.85 1.85) (drill 0.9) (layers *.Cu *.Mask) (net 11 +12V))
  (pad 2 thru_hole circle (at 2.5 0 270) (size 1.85 1.85) (drill 0.9) (layers *.Cu *.Mask) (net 1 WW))
  (pad 3 thru_hole circle (at 5 0 270) (size 1.85 1.85) (drill 0.9) (layers *.Cu *.Mask) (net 5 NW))
  (pad 4 thru_hole circle (at 7.5 0 270) (size 1.85 1.85) (drill 0.9) (layers *.Cu *.Mask) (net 9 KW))
  (pad 5 thru_hole circle (at 10 0 270) (size 1.85 1.85) (drill 0.9) (layers *.Cu *.Mask) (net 30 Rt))
  (pad 6 thru_hole circle (at 12.5 0 270) (size 1.85 1.85) (drill 0.9) (layers *.Cu *.Mask) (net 32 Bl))
  (pad 7 thru_hole circle (at 15 0 270) (size 1.85 1.85) (drill 0.9) (layers *.Cu *.Mask) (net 2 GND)))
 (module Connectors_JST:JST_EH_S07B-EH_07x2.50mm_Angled (layer B.Cu) (at 202.5 71.5 90)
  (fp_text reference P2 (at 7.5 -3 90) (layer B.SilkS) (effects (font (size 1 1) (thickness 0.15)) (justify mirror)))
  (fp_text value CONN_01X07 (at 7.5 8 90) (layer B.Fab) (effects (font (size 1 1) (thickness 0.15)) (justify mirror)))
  (pad 1 thru_hole rect (at 0 0 90) (size 1.85 1.85) (drill 0.9) (layers *.Cu *.Mask) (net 11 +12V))
  (pad 2 thru_hole circle (at 2.5 0 90) (size 1.85 1.85) (drill 0.9) (layers *.Cu *.Mask) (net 1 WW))
  (pad 3 thru_hole circle (at 5 0 90) (size 1.85 1.85) (drill 0.9) (layers *.Cu *.Mask) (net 5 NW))
  (pad 4 thru_hole circle (at 7.5 0 90) (size 1.85 1.85) (drill 0.9) (layers *.Cu *.Mask) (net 9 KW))
  (pad 5 thru_hole circle (at 10 0 90) (size 1.85 1.85) (drill 0.9) (layers *.Cu *.Mask) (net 30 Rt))
  (pad 6 thru_hole circle (at 12.5 0 90) (size 1.85 1.85) (drill 0.9) (layers *.Cu *.Mask) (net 32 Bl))
  (pad 7 thru_hole circle (at 15 0 90) (size 1.85 1.85) (drill 0.9) (layers *.Cu *.Mask) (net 2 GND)))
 (gr_line (start 113.5 89.5) (end 205.5 89.5) (angle 90) (layer Edge.Cuts) (width 0.15))
 (gr_line (start 109.5 43.5) (end 109.5 85.5) (angle 90) (layer Edge.Cuts) (width 0.15))
 (gr_line (start 205.5 39.5) (end 113.5 39.5) (angle 90) (layer Edge.Cuts) (width 0.15))
 (gr_line (start 209.5 85.5) (end 209.5 43.5) (angle 90) (layer Edge.Cuts) (width 0.15))
 (gr_arc (start 205.5 43.5) (end 205.5 39.5) (angle 90) (layer Edge.Cuts) (width 0.15))
 (gr_arc (start 205.5 85.5) (end 209.5 85.5) (angle 90) (layer Edge.Cuts) (width 0.15))
 (gr_arc (start 113.5 85.5) (end 113.5 89.5) (angle 90) (layer Edge.Cuts) (width 0.15))
 (gr_arc (start 113.5 43.5) (end 109.5 43.5) (angle 90) (layer Edge.Cuts) (width 0.15))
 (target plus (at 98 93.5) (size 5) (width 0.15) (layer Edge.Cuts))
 (segment (start 129 87.5) (end 129 86.75) (width 0.4) (layer F.Cu) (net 2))
 (segment (start 129.2 86.55) (end 129.2 85.5) (width 0.4) (layer F.Cu) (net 2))
 (segment (start 129 86.75) (end 129.2 86.55) (width 0.4) (layer F.Cu) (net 2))
 (segment (start 129.2 85.5) (end 130.5 85.5) (width 0.4) (layer F.Cu) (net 2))
 (via (at 130.5 85.5) (size 0.6) (drill 0.4) (layers F.Cu B.Cu) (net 2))
 (segment (start 141.5 87.5) (end 141.5 85.7) (width 0.4) (layer F.Cu) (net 2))
 (segment (start 141.5 85.7) (end 141.7 85.5) (width 0.4) (layer F.Cu) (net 2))
 (segment (start 141.7 85.5) (end 143 85.5) (width 0.4) (layer F.Cu) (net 2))
 (via (at 143 85.5) (size 0.6) (drill 0.4) (layers F.Cu B.Cu) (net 2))
 (segment (start 154 87.5) (end 154 86.75) (width 0.4) (layer F.Cu) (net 2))
 (segment (start 154.2 86.55) (end 154.2 85.5) (width 0.4) (layer F.Cu) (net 2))
 (segment (start 154 86.75) (end 154.2 86.55) (width 0.4) (layer F.Cu) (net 2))
 (segment (start 154.2 85.5) (end 155.5 85.5) (width 0.4) (layer F.Cu) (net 2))
 (via (at 155.5 85.5) (size 0.6) (drill 0.4) (layers F.Cu B.Cu) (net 2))
 (segment (start 165.25 87.5) (end 165.25 86.5) (width 0.4) (layer F.Cu) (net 2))
 (segment (start 165.45 86.3) (end 165.45 85.5) (width 0.4) (layer F.Cu) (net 2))
 (segment (start 165.25 86.5) (end 165.45 86.3) (width 0.4) (layer F.Cu) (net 2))
 (segment (start 165.45 85.5) (end 166.5 85.5) (width 0.4) (layer F.Cu) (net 2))
 (via (at 166.5 85.5) (size 0.6) (drill 0.4) (layers F.Cu B.Cu) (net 2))
 (segment (start 166.5 85.5) (end 166.75 85.5) (width 0.4) (layer B.Cu) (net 2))
 (segment (start 179.2 85.5) (end 180.5 85.5) (width 0.4) (layer F.Cu) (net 2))
 (via (at 180.5 85.5) (size 0.6) (drill 0.4) (layers F.Cu B.Cu) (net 2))
 (segment (start 179 87.5) (end 179 85.7) (width 0.4) (layer F.Cu) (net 2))
 (segment (start 179 85.7) (end 179.2 85.5) (width 0.4) (layer F.Cu) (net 2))
 (segment (start 191.5 87.5) (end 191.5 86.5) (width 0.4) (layer F.Cu) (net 2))
 (segment (start 191.7 86.3) (end 191.7 85.5) (width 0.4) (layer F.Cu) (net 2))
 (segment (start 191.5 86.5) (end 191.7 86.3) (width 0.4) (layer F.Cu) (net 2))
 (segment (start 191.7 85.5) (end 194.25 85.5) (width 0.4) (layer F.Cu) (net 2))
 (via (at 194.25 85.5) (size 0.6) (drill 0.4) (layers F.Cu B.Cu) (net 2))
 (segment (start 202.5 56.5) (end 199.75 59.25) (width 0.75) (layer B.Cu) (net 2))
 (segment (start 130.5 85.5) (end 116.5 71.5) (width 0.75) (layer B.Cu) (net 2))
 (segment (start 180.5 85.5) (end 166.75 85.5) (width 0.75) (layer B.Cu) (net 2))
 (segment (start 166.75 85.5) (end 155.5 85.5) (width 0.75) (layer B.Cu) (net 2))
 (segment (start 155.5 85.5) (end 143 85.5) (width 0.75) (layer B.Cu) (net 2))
 (segment (start 143 85.5) (end 130.5 85.5) (width 0.75) (layer B.Cu) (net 2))
 (segment (start 194.25 85.5) (end 180.5 85.5) (width 0.75) (layer B.Cu) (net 2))
 (segment (start 199.75 80) (end 194.25 85.5) (width 0.75) (layer B.Cu) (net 2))
 (segment (start 199.75 59.25) (end 199.75 80) (width 0.75) (layer B.Cu) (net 2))
 (segment (start 202.5 56.5) (end 202.5 49.25) (width 0.75) (layer B.Cu) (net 2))
 (segment (start 202.05 48.8) (end 203.25 48.8) (width 0.75) (layer F.Cu) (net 2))
 (segment (start 201.25 48) (end 202.05 48.8) (width 0.75) (layer F.Cu) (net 2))
 (via (at 201.25 48) (size 0.6) (drill 0.4) (layers F.Cu B.Cu) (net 2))
 (segment (start 202.5 49.25) (end 201.25 48) (width 0.75) (layer B.Cu) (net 2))
 (segment (start 203.25 48.8) (end 203.45 49) (width 0.75) (layer F.Cu) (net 2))
 (segment (start 203.45 49) (end 205.75 49) (width 0.75) (layer F.Cu) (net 2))
 (segment (start 115.05 78) (end 113.5 76.45) (width 0.75) (layer F.Cu) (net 11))
 (segment (start 113.5 59.5) (end 116.5 56.5) (width 0.75) (layer F.Cu) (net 11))
 (segment (start 113.5 76.45) (end 113.5 59.5) (width 0.75) (layer F.Cu) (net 11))
 (segment (start 116.5 56.5) (end 116.5 51.45) (width 0.75) (layer F.Cu) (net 11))
 (segment (start 116.5 51.45) (end 115.05 50) (width 0.75) (layer F.Cu) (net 11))
 (segment (start 115.05 50) (end 115.05 48.45) (width 0.75) (layer F.Cu) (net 11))
 (segment (start 115.05 48.45) (end 121.45 42.05) (width 0.75) (layer F.Cu) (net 11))
 (segment (start 121.45 42.05) (end 128.25 42.05) (width 0.75) (layer F.Cu) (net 11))
 (segment (start 128.25 42.05) (end 140.75 42.05) (width 0.75) (layer F.Cu) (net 11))
 (segment (start 140.75 42.05) (end 153.25 42.05) (width 0.75) (layer F.Cu) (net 11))
 (segment (start 153.25 42.05) (end 178.25 42.05) (width 0.75) (layer F.Cu) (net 11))
 (segment (start 178.25 42.05) (end 190.75 42.05) (width 0.75) (layer F.Cu) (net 11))
 (segment (start 190.75 42.05) (end 197.8 42.05) (width 0.75) (layer F.Cu) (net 11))
 (segment (start 197.8 42.05) (end 200.75 45) (width 0.75) (layer F.Cu) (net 11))
 (via (at 200.75 45) (size 0.6) (drill 0.4) (layers F.Cu B.Cu) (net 11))
 (segment (start 200.75 45) (end 205.25 49.5) (width 0.75) (layer B.Cu) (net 11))
 (segment (start 205.25 49.5) (end 205.25 68.75) (width 0.75) (layer B.Cu) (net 11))
 (segment (start 205.25 68.75) (end 202.5 71.5) (width 0.75) (layer B.Cu) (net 11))
 (segment (start 202.5 61.5) (end 204.25 59.75) (width 0.4) (layer B.Cu) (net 30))
 (segment (start 204 51.45) (end 203.25 50.7) (width 0.4) (layer F.Cu) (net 30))
 (segment (start 204 52.25) (end 204 51.45) (width 0.4) (layer F.Cu) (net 30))
 (via (at 204 52.25) (size 0.6) (drill 0.4) (layers F.Cu B.Cu) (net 30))
 (segment (start 204.25 52.5) (end 204 52.25) (width 0.4) (layer B.Cu) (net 30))
 (segment (start 204.25 59.75) (end 204.25 52.5) (width 0.4) (layer B.Cu) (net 30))
 (segment (start 205.75 50.5) (end 204.75 50.5) (width 0.4) (layer F.Cu) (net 30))
 (segment (start 204.55 50.7) (end 203.25 50.7) (width 0.4) (layer F.Cu) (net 30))
 (segment (start 204.75 50.5) (end 204.55 50.7) (width 0.4) (layer F.Cu) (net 30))
 (segment (start 202.5 59) (end 207 63.5) (width 0.4) (layer F.Cu) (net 32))
 (segment (start 206 79) (end 205 79) (width 0.4) (layer F.Cu) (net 32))
 (segment (start 207 78) (end 206 79) (width 0.4) (layer F.Cu) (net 32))
 (segment (start 207 63.5) (end 207 78) (width 0.4) (layer F.Cu) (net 32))
 (segment (start 205 79) (end 204 79) (width 0.4) (layer F.Cu) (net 32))
 (segment (start 204 79) (end 203.2 79) (width 0.4) (layer F.Cu) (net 32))
 (segment (start 203.2 79) (end 203 79.2) (width 0.4) (layer F.Cu) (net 32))
 (segment (start 117.95 50) (end 120 50) (width 0.4) (layer F.Cu) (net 34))
 (segment (start 131.25 57.75) (end 133.525 57.75) (width 0.4) (layer F.Cu) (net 34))
 (via (at 131.25 57.75) (size 0.6) (drill 0.4) (layers F.Cu B.Cu) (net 34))
 (segment (start 127.75 57.75) (end 131.25 57.75) (width 0.4) (layer B.Cu) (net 34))
 (segment (start 120 50) (end 127.75 57.75) (width 0.4) (layer B.Cu) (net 34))
 (via (at 120 50) (size 0.6) (drill 0.4) (layers F.Cu B.Cu) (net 34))
 (segment (start 136 57.75) (end 138 57.75) (width 0.4) (layer F.Cu) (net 36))
 (segment (start 156.25 57.75) (end 158.525 57.75) (width 0.4) (layer F.Cu) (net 36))
 (via (at 156.25 57.75) (size 0.6) (drill 0.4) (layers F.Cu B.Cu) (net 36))
 (segment (start 138 57.75) (end 156.25 57.75) (width 0.4) (layer B.Cu) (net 36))
 (via (at 138 57.75) (size 0.6) (drill 0.4) (layers F.Cu B.Cu) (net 36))
 (segment (start 135.475 70.25) (end 138 70.25) (width 0.4) (layer F.Cu) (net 38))
 (segment (start 156 70.25) (end 158 70.25) (width 0.4) (layer F.Cu) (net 38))
 (via (at 156 70.25) (size 0.6) (drill 0.4) (layers F.Cu B.Cu) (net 38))
 (segment (start 138 70.25) (end 156 70.25) (width 0.4) (layer B.Cu) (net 38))
 (via (at 138 70.25) (size 0.6) (drill 0.4) (layers F.Cu B.Cu) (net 38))
 (via (at 131.5 70.25) (size 0.6) (drill 0.4) (layers F.Cu B.Cu) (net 35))
 (segment (start 126.5 70.25) (end 131.5 70.25) (width 0.4) (layer B.Cu) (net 35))
 (via (at 126.5 70.25) (size 0.6) (drill 0.4) (layers F.Cu B.Cu) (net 35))
 (segment (start 118.75 78) (end 126.5 70.25) (width 0.4) (layer F.Cu) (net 35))
 (segment (start 117.95 78) (end 118.75 78) (width 0.4) (layer F.Cu) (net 35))
 (segment (start 131.5 70.25) (end 133 70.25) (width 0.4) (layer F.Cu) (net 35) (status 800000))
 (segment (start 160.475 70.25) (end 162.75 70.25) (width 0.4) (layer F.Cu) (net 39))
 (segment (start 181 70.25) (end 183 70.25) (width 0.4) (layer F.Cu) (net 39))
 (via (at 181 70.25) (size 0.6) (drill 0.4) (layers F.Cu B.Cu) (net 39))
 (segment (start 162.75 70.25) (end 181 70.25) (width 0.4) (layer B.Cu) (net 39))
 (via (at 162.75 70.25) (size 0.6) (drill 0.4) (layers F.Cu B.Cu) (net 39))
 (segment (start 185.475 70.25) (end 188.25 70.25) (width 0.4) (layer F.Cu) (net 33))
 (segment (start 200 78.25) (end 201 78.25) (width 0.4) (layer F.Cu) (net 33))
 (segment (start 198.75 77) (end 200 78.25) (width 0.4) (layer F.Cu) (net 33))
 (segment (start 198.75 72.25) (end 198.75 77) (width 0.4) (layer F.Cu) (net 33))
 (segment (start 196.75 70.25) (end 198.75 72.25) (width 0.4) (layer F.Cu) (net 33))
 (via (at 196.75 70.25) (size 0.6) (drill 0.4) (layers F.Cu B.Cu) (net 33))
 (segment (start 188.25 70.25) (end 196.75 70.25) (width 0.4) (layer B.Cu) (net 33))
 (via (at 188.25 70.25) (size 0.6) (drill 0.4) (layers F.Cu B.Cu) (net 33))
 (segment (start 161 57.75) (end 163 57.75) (width 0.4) (layer F.Cu) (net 37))
 (segment (start 181 57.75) (end 183.525 57.75) (width 0.4) (layer F.Cu) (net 37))
 (via (at 181 57.75) (size 0.6) (drill 0.4) (layers F.Cu B.Cu) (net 37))
 (segment (start 163 57.75) (end 181 57.75) (width 0.4) (layer B.Cu) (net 37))
 (via (at 163 57.75) (size 0.6) (drill 0.4) (layers F.Cu B.Cu) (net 37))
 (segment (start 186 57.75) (end 188 57.75) (width 0.4) (layer F.Cu) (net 31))
 (segment (start 200 49.75) (end 201.25 49.75) (width 0.4) (layer F.Cu) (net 31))
 (via (at 200 49.75) (size 0.6) (drill 0.4) (layers F.Cu B.Cu) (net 31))
 (segment (start 192 57.75) (end 200 49.75) (width 0.4) (layer B.Cu) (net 31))
 (segment (start 188 57.75) (end 192 57.75) (width 0.4) (layer B.Cu) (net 31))
 (via (at 188 57.75) (size 0.6) (drill 0.4) (layers F.Cu B.Cu) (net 31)))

